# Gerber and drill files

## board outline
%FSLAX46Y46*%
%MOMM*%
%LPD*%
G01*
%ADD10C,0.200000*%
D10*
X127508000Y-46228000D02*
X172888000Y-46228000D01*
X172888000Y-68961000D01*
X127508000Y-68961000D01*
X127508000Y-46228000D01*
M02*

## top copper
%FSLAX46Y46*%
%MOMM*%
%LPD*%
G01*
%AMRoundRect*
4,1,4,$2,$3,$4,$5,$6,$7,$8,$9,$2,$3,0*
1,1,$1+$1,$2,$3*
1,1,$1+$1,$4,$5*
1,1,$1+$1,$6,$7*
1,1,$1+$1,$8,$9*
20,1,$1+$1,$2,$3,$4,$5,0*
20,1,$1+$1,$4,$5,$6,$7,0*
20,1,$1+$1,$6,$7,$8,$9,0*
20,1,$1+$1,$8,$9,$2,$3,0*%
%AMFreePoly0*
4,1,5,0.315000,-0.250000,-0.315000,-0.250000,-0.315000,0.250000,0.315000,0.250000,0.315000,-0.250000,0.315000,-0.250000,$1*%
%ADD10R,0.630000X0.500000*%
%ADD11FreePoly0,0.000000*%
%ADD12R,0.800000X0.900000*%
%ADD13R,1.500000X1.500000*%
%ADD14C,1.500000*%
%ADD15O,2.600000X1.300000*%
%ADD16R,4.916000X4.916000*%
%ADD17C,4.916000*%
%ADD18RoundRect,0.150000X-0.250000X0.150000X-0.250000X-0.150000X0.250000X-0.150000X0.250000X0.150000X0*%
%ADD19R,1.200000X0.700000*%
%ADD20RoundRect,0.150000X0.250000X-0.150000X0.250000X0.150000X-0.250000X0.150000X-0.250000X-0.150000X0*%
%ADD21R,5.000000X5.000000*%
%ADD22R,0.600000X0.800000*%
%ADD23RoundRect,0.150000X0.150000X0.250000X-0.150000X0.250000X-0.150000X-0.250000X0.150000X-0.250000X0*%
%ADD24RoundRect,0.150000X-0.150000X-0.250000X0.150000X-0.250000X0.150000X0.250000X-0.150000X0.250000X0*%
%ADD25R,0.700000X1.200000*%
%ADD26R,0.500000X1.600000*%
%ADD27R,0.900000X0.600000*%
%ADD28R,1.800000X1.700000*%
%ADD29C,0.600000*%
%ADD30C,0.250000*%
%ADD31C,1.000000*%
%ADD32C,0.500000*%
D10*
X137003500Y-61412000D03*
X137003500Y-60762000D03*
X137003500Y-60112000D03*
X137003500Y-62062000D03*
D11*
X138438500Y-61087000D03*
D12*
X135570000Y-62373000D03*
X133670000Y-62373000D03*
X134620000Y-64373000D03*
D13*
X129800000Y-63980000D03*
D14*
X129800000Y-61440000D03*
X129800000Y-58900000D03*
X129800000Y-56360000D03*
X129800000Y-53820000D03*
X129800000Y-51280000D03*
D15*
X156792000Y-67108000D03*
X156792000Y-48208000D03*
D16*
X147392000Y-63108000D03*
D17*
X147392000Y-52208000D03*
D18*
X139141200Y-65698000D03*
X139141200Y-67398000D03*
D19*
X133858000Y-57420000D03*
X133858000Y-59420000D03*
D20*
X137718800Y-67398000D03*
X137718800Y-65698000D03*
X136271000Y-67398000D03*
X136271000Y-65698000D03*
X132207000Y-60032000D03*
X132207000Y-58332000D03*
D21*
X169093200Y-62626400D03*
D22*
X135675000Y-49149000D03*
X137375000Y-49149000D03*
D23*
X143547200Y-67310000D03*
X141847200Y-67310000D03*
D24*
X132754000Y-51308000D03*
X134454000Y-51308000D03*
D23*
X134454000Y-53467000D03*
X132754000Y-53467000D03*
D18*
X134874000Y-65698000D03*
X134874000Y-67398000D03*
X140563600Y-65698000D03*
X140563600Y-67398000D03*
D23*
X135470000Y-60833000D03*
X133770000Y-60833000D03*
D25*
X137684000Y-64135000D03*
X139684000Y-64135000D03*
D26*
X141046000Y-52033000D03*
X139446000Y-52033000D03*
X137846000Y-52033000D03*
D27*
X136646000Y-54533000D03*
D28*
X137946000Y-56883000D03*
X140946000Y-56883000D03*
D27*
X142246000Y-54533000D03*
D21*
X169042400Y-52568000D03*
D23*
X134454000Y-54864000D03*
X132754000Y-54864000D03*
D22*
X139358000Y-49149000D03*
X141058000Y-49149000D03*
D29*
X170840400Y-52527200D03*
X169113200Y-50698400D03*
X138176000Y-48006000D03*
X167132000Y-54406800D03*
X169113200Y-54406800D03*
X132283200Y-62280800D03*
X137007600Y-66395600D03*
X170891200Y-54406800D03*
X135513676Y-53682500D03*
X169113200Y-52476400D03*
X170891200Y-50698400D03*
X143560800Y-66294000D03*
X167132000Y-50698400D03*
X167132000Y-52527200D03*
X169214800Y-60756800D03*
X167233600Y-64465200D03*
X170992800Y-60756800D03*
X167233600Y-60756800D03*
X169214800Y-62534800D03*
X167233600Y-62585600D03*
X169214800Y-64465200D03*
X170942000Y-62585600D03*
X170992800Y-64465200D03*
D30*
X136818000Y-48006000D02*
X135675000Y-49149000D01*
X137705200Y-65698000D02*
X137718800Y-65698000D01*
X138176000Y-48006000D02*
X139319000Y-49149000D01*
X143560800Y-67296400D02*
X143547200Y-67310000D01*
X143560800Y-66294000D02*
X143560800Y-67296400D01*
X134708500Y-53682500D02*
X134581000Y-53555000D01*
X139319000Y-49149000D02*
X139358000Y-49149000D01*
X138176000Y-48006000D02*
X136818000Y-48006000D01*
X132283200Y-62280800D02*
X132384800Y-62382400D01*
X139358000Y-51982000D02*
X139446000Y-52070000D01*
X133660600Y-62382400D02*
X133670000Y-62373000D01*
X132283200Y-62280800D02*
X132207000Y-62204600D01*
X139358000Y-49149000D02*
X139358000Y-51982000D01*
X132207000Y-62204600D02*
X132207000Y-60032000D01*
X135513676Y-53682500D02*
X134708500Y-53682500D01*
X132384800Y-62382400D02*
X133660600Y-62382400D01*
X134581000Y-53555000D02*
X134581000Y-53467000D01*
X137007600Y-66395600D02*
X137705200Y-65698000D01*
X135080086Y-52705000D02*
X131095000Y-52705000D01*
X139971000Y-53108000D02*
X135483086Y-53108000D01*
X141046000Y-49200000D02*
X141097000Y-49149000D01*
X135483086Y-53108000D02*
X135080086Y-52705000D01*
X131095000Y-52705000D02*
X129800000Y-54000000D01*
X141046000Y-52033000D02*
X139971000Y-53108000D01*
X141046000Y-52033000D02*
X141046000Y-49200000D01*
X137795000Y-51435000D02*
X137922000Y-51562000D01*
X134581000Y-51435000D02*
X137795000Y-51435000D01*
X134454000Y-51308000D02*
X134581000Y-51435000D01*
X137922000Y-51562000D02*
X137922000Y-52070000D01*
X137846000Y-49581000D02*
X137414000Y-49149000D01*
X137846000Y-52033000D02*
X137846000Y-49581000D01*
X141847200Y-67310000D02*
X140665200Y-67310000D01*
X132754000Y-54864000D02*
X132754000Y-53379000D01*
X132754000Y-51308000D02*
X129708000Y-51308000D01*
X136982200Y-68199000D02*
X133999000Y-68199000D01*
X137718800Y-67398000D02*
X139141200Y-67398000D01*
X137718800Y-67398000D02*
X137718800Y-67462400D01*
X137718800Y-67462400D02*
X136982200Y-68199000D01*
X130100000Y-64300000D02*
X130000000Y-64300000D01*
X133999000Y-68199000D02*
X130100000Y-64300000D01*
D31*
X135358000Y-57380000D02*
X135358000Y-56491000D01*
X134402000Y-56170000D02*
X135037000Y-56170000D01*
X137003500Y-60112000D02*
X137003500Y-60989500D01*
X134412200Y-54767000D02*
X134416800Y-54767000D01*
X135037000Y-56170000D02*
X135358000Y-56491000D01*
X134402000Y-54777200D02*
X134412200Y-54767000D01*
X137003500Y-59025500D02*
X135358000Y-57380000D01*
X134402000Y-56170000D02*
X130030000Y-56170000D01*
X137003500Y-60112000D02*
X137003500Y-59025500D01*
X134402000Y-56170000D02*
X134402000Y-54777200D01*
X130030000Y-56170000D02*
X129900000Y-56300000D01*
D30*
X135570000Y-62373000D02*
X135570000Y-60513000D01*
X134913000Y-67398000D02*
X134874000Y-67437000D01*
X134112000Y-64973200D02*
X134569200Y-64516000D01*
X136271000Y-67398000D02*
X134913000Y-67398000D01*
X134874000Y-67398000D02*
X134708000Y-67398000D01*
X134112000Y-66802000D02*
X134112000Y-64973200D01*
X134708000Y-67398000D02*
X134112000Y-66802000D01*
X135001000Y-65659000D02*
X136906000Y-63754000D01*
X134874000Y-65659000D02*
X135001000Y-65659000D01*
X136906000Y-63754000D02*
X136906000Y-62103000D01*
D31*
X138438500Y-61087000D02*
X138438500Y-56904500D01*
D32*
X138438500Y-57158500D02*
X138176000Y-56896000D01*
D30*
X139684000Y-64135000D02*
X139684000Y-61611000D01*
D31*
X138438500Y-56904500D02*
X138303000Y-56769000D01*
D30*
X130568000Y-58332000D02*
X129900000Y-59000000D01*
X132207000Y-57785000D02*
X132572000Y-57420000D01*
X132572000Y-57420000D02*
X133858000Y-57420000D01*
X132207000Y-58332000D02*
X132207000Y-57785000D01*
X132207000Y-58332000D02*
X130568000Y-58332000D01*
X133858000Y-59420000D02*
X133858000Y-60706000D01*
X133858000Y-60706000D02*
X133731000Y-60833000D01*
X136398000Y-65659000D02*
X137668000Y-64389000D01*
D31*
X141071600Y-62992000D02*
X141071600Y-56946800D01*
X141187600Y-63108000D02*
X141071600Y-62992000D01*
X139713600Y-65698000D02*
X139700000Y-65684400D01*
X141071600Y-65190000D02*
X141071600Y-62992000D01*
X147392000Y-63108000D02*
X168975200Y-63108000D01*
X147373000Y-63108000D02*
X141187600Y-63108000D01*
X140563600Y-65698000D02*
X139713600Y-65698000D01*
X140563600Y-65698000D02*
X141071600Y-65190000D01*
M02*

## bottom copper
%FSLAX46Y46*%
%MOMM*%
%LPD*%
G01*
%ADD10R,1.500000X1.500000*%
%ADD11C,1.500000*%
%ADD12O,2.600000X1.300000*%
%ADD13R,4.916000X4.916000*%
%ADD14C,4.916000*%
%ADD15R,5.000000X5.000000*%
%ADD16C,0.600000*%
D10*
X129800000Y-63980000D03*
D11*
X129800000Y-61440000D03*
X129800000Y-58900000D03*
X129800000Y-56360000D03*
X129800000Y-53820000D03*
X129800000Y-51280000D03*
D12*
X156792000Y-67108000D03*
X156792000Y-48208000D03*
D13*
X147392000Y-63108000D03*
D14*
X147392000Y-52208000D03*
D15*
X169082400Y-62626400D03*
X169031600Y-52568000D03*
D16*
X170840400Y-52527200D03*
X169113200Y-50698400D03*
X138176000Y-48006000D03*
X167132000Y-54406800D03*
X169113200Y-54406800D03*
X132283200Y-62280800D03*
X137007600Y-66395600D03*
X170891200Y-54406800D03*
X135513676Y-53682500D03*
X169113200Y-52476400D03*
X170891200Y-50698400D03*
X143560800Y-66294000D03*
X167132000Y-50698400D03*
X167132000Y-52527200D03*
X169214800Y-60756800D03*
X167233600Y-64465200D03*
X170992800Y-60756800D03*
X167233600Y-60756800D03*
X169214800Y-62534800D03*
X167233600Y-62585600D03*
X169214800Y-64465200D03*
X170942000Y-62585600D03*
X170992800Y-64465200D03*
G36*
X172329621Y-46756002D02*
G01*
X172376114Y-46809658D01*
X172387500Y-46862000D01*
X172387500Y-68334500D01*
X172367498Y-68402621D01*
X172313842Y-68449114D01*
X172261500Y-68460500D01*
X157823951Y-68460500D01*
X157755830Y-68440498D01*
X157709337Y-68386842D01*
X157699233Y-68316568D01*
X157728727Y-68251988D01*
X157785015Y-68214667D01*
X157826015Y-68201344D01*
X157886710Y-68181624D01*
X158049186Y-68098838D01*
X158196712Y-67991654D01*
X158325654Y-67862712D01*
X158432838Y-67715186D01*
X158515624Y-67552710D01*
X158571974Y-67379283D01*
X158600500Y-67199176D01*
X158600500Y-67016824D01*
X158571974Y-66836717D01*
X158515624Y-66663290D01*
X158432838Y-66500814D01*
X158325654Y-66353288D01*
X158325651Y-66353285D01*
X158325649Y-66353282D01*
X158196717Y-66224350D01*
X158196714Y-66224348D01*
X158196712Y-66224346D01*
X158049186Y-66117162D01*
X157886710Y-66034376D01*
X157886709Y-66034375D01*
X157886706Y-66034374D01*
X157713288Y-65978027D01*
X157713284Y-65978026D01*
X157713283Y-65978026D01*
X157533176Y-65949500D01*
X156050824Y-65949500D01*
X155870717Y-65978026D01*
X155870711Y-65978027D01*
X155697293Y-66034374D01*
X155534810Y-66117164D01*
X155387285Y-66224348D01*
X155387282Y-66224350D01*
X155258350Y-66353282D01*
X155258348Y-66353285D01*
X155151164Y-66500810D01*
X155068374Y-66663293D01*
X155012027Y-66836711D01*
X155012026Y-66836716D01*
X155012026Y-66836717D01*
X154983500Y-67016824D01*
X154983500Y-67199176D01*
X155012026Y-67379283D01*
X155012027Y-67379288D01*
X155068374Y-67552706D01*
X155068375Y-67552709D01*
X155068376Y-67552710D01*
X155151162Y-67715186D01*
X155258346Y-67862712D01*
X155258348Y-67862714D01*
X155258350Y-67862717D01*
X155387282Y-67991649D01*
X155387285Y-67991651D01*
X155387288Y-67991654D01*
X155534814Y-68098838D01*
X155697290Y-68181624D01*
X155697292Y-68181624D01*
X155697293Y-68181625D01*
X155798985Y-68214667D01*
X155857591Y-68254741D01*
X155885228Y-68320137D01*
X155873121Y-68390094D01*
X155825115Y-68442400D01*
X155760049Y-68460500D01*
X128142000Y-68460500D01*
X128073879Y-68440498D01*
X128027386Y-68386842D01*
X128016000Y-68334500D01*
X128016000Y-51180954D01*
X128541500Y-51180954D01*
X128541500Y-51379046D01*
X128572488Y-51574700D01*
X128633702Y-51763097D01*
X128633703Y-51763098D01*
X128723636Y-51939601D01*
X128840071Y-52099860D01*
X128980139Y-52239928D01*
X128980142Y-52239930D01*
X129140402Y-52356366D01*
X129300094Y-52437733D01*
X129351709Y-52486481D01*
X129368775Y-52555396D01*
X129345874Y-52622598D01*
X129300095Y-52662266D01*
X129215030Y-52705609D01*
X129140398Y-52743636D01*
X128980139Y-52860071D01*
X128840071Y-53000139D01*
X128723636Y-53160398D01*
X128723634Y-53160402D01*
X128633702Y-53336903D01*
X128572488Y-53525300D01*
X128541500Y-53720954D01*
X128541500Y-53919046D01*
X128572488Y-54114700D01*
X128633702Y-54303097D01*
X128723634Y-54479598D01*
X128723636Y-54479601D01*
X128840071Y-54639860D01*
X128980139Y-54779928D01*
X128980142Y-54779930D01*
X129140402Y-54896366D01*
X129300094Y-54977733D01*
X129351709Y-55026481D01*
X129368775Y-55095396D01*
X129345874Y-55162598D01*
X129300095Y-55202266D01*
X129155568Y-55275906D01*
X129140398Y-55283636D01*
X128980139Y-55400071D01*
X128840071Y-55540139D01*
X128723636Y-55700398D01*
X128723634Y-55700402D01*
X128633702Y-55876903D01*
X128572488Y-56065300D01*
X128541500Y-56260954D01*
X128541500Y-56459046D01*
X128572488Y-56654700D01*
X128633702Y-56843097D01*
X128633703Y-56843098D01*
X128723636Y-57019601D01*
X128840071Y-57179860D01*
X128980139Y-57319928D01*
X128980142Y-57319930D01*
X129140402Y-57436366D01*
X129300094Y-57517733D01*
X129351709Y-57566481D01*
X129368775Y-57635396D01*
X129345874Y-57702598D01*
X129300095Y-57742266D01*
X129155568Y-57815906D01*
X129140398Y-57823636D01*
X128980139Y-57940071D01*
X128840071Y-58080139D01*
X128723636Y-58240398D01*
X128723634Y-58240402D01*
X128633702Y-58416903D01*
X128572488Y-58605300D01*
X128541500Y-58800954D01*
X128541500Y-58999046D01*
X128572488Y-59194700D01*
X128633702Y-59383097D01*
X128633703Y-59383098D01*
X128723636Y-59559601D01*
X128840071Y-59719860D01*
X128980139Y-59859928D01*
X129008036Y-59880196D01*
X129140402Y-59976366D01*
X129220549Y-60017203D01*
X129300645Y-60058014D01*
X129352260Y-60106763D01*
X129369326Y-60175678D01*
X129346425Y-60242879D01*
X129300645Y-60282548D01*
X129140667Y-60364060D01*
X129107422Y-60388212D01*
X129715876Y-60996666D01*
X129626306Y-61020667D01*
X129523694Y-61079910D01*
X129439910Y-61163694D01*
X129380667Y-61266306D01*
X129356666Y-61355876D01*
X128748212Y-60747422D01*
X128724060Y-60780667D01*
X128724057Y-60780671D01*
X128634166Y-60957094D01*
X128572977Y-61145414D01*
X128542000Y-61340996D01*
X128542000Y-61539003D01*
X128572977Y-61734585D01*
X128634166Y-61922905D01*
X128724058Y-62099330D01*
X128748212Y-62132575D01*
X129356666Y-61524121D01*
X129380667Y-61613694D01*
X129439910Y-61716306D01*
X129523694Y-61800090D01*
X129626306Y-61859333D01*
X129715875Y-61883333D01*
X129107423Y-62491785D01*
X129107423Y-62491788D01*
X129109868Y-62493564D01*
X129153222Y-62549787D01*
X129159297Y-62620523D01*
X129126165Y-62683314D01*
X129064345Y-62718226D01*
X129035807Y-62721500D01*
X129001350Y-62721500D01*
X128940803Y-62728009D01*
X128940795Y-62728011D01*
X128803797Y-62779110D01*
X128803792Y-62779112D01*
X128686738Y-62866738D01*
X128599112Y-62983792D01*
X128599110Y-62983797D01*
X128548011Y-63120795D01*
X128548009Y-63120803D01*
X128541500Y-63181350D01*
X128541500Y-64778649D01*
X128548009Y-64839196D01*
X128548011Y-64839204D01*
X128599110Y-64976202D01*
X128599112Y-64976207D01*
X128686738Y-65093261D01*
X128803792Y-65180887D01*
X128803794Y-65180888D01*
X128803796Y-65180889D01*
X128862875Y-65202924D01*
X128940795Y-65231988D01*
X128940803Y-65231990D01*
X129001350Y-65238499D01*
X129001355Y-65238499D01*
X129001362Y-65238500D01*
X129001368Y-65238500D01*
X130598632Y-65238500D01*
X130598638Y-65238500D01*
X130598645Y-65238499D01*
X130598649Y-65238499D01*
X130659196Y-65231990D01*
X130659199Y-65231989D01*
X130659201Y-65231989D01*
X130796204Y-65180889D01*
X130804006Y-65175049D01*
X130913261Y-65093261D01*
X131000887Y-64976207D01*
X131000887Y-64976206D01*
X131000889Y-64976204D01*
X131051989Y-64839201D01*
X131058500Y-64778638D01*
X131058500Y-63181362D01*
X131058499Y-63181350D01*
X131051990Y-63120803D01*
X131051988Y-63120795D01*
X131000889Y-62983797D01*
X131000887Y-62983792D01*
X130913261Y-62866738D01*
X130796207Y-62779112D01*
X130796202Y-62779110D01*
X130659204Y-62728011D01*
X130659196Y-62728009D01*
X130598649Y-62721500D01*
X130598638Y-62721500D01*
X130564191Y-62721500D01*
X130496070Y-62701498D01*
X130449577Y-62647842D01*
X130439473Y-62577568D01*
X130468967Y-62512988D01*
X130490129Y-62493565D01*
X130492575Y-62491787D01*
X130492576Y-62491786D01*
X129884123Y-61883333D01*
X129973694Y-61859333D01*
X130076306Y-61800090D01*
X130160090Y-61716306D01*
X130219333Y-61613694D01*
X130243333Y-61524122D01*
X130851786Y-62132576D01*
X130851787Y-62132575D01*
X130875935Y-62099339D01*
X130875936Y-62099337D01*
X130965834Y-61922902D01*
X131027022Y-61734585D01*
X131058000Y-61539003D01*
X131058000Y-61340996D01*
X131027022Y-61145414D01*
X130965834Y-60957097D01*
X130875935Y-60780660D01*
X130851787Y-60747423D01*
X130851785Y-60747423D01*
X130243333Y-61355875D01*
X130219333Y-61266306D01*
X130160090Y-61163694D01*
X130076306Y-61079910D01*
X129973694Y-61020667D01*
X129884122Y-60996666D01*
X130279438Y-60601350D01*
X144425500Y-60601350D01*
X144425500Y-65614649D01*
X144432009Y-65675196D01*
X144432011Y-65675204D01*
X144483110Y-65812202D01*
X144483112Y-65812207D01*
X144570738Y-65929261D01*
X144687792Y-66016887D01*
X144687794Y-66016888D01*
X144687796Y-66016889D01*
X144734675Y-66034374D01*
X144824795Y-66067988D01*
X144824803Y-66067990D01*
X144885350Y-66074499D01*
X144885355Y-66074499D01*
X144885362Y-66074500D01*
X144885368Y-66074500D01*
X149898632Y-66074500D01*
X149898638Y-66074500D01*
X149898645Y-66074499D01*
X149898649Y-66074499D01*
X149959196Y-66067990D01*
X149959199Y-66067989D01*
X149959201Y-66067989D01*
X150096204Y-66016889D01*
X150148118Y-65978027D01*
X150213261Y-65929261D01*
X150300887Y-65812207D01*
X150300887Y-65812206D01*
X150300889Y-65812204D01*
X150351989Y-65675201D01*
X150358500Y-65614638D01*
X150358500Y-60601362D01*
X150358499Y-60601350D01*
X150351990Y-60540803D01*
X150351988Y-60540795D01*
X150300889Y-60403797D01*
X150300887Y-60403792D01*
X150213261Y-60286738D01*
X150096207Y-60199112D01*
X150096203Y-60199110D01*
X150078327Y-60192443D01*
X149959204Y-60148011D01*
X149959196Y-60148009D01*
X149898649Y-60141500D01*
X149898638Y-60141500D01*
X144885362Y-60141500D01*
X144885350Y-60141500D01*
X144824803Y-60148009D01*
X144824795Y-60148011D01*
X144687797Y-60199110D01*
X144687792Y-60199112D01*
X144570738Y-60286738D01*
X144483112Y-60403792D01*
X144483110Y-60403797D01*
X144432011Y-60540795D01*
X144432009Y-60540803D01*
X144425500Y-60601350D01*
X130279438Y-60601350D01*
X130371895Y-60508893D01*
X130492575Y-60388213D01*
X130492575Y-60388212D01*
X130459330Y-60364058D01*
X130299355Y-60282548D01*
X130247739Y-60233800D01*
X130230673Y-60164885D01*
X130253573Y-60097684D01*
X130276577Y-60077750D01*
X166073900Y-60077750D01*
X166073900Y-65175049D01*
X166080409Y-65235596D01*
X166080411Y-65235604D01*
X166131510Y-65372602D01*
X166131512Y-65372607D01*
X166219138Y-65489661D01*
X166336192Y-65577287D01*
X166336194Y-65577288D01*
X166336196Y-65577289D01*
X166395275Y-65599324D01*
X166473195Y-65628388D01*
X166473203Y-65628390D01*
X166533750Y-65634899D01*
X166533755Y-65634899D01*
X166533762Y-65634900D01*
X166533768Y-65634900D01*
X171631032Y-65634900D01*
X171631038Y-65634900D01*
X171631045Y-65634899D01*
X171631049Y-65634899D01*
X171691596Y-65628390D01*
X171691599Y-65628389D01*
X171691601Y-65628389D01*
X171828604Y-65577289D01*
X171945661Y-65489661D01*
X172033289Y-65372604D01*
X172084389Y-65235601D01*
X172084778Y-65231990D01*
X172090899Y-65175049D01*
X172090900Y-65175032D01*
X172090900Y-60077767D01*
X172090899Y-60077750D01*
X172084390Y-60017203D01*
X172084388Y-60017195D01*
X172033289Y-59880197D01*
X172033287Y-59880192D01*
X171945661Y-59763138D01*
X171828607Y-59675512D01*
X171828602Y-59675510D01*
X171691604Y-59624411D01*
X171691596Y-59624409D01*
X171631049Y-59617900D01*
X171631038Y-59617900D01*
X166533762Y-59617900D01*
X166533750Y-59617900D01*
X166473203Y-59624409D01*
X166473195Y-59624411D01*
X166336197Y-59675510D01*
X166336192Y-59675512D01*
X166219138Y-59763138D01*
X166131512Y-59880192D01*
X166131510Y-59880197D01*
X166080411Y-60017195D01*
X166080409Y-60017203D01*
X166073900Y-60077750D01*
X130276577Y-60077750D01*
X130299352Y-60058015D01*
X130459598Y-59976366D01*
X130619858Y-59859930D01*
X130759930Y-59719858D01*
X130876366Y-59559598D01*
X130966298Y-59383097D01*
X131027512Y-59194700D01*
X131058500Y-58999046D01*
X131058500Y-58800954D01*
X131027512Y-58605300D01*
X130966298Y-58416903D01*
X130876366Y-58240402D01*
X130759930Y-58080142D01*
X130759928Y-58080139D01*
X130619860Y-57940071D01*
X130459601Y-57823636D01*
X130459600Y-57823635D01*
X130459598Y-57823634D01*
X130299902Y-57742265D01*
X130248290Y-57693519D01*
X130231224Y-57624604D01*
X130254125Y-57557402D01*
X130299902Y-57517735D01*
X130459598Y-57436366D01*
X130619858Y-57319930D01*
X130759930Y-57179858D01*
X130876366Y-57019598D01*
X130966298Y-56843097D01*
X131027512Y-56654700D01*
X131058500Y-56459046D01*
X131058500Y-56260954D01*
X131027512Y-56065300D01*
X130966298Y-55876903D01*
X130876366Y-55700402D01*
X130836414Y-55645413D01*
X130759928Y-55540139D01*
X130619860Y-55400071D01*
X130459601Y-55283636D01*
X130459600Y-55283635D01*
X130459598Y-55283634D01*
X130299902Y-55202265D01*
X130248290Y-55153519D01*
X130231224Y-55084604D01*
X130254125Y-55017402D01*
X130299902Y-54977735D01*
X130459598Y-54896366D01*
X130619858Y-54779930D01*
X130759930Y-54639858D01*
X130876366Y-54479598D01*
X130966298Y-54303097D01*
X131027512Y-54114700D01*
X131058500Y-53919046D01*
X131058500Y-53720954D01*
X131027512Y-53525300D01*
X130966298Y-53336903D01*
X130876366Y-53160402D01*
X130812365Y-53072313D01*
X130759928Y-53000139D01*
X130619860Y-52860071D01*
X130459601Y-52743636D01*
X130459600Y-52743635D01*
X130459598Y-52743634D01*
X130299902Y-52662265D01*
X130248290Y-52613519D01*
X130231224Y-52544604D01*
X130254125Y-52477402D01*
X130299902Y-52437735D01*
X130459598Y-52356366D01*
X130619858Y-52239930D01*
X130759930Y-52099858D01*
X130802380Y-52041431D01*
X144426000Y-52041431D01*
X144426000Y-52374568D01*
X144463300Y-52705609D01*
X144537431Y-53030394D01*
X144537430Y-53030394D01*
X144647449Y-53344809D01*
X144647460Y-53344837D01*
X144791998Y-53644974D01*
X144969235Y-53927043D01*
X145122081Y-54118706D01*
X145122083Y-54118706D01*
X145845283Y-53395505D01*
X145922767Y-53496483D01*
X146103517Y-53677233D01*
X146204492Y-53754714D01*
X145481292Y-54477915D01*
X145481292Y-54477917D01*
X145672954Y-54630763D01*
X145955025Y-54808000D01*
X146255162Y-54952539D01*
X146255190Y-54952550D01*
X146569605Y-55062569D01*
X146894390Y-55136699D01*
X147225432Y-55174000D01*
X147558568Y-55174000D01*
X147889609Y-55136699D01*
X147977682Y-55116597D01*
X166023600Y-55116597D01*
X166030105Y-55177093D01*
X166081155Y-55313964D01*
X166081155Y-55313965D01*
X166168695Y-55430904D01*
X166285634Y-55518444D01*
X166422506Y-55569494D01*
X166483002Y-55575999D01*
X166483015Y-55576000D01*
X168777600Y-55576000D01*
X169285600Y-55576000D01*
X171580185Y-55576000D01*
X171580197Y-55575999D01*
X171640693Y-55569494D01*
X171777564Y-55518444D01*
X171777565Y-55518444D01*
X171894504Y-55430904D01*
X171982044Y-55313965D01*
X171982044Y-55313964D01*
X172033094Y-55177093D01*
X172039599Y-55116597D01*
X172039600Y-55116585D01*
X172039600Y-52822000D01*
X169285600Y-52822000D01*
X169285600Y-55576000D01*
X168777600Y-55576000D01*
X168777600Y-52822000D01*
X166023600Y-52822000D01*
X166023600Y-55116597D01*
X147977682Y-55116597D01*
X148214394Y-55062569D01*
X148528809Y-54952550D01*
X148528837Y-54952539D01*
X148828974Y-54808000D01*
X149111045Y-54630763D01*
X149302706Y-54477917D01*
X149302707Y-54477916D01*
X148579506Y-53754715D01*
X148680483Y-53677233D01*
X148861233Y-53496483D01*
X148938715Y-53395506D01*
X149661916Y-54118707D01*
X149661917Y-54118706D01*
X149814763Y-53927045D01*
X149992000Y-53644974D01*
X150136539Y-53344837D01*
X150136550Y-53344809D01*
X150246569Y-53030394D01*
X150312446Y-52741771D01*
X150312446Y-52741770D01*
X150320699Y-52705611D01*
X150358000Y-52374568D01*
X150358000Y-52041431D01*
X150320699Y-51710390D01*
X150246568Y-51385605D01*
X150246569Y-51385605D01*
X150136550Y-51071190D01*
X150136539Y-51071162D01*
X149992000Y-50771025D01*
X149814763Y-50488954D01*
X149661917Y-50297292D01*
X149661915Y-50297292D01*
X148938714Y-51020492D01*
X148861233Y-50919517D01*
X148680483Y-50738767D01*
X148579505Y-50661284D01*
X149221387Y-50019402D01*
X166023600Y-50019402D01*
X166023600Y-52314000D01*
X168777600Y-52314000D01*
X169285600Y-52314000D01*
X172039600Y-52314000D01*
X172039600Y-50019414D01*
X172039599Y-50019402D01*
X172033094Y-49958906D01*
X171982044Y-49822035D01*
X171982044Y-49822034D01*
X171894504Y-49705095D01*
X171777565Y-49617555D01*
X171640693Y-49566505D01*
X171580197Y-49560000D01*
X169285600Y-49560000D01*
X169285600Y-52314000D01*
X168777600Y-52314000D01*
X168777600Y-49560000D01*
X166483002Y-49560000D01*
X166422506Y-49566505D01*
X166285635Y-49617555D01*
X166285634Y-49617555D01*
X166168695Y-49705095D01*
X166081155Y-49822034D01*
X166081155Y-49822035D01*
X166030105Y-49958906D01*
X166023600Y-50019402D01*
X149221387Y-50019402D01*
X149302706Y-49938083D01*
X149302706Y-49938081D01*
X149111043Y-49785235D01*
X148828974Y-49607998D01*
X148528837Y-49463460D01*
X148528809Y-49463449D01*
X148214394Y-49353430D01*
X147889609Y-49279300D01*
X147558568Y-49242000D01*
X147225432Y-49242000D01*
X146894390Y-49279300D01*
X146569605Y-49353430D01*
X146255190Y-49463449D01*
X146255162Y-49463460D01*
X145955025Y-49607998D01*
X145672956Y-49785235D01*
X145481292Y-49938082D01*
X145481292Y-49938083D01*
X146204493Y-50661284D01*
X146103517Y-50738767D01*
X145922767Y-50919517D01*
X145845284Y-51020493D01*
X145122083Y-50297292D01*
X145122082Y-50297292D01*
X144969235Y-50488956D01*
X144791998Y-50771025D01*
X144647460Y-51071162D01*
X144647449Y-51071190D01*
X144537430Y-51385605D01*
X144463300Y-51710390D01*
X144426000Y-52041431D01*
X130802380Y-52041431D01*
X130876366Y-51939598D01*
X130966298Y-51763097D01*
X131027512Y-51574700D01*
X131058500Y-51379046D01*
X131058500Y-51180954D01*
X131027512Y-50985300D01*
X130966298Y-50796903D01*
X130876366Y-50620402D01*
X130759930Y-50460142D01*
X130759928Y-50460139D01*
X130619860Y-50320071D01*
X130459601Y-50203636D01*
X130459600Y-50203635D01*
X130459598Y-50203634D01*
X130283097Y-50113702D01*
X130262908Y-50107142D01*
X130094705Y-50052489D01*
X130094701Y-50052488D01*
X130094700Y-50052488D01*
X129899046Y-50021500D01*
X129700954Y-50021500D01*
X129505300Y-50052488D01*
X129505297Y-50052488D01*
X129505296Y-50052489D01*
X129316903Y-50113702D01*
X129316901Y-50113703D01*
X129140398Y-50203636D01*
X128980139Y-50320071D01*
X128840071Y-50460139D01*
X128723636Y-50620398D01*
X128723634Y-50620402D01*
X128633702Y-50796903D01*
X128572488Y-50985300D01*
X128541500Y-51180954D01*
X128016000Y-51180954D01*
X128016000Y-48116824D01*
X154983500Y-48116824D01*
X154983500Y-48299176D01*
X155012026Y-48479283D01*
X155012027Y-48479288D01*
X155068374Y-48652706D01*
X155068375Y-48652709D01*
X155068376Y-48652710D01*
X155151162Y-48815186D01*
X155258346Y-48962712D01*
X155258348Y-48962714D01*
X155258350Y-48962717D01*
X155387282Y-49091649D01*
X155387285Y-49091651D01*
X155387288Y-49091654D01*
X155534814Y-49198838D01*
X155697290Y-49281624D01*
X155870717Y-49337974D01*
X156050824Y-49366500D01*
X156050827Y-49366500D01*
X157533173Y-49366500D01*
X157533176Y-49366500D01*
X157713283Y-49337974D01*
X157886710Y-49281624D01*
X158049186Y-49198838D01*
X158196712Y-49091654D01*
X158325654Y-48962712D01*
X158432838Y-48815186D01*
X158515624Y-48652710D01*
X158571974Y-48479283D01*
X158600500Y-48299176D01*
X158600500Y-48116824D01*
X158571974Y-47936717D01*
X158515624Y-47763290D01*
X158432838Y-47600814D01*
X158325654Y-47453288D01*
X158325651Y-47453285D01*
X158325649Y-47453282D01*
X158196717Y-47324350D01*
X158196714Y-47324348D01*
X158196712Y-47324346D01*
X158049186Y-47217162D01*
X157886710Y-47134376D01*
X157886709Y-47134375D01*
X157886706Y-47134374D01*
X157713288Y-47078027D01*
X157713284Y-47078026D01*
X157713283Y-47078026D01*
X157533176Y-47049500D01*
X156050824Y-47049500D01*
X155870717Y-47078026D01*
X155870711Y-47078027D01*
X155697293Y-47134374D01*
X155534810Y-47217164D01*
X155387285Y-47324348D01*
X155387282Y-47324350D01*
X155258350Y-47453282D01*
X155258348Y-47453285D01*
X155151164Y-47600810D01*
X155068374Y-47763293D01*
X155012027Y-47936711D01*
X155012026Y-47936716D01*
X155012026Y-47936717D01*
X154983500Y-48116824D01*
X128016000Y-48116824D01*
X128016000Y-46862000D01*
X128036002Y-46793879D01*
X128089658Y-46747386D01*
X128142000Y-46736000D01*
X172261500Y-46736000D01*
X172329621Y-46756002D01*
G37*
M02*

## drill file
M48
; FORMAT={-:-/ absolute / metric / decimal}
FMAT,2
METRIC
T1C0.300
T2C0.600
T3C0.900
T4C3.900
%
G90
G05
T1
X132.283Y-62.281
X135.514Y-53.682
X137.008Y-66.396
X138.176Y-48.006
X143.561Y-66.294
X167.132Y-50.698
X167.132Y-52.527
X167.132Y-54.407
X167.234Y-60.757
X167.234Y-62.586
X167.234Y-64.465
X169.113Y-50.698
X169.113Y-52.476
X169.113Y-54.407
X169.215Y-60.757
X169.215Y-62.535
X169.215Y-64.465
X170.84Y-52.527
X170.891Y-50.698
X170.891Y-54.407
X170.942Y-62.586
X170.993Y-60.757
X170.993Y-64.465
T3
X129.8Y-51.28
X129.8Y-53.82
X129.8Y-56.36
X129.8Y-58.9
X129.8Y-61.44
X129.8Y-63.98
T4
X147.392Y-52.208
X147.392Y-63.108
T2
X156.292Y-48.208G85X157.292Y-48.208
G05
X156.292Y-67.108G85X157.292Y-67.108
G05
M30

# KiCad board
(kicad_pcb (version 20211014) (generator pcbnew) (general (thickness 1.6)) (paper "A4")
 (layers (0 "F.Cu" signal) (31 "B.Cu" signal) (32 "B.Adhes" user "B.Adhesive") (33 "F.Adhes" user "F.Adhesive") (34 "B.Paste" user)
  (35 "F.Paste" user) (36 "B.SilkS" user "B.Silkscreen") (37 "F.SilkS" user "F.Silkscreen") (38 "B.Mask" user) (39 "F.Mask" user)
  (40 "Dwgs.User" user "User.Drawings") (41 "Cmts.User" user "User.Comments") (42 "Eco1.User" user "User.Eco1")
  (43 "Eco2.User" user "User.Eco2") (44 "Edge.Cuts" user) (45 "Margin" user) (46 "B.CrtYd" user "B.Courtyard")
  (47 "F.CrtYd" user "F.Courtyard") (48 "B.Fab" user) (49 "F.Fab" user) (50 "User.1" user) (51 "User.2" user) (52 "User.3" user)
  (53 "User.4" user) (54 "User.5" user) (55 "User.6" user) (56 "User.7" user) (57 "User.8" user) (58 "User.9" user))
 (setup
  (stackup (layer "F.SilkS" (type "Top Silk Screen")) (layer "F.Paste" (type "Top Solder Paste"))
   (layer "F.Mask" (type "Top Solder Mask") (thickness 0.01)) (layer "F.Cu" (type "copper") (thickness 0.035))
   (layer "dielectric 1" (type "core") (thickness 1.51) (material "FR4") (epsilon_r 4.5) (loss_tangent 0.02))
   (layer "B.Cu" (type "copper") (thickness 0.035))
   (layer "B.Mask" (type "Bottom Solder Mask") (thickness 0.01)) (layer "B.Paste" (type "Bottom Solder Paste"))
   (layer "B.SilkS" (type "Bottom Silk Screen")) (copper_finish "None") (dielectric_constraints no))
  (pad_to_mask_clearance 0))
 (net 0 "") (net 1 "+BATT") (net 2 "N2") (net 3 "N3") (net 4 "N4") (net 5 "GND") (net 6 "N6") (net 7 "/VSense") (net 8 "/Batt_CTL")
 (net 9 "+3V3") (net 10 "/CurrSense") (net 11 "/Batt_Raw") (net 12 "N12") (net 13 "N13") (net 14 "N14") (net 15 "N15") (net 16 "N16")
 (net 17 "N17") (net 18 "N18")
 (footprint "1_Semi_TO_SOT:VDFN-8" (layer "F.Cu") (at 138.4385 61.087) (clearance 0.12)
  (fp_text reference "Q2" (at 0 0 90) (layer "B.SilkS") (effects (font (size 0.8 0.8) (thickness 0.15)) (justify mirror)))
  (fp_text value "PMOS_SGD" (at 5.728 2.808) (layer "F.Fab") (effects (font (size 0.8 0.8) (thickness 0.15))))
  (pad "1" smd rect (at -1.435 0.325) (size 0.63 0.5) (layers "F.Cu" "F.Mask") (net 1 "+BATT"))
  (pad "1" smd rect (at -1.435 -0.325) (size 0.63 0.5) (layers "F.Cu" "F.Mask") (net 1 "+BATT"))
  (pad "1" smd rect (at -1.435 -0.975) (size 0.63 0.5) (layers "F.Cu" "F.Mask") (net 1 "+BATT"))
  (pad "2" smd rect (at -1.435 0.975) (size 0.63 0.5) (layers "F.Cu" "F.Mask") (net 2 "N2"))
  (pad "3" smd custom (at 0 0) (size 0.63 0.5) (layers "F.Cu") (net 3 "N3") (zone_connect 0) (options (clearance outline) (anchor rect))
   (primitives)))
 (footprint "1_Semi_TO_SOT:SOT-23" (layer "F.Cu") (at 134.62 63.373 -90)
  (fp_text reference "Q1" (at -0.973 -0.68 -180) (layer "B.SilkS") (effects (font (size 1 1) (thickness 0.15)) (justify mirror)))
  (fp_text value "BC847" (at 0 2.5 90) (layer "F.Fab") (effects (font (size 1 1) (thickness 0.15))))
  (pad "1" smd rect locked (at -1 -0.95 270) (size 0.9 0.8) (layers "F.Cu" "F.Paste" "F.Mask") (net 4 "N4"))
  (pad "2" smd rect locked (at -1 0.95 270) (size 0.9 0.8) (layers "F.Cu" "F.Paste" "F.Mask") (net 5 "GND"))
  (pad "3" smd rect locked (at 1 0 270) (size 0.9 0.8) (layers "F.Cu" "F.Paste" "F.Mask") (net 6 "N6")))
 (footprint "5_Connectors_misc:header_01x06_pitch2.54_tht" (layer "F.Cu") (at 129.8 63.98 90)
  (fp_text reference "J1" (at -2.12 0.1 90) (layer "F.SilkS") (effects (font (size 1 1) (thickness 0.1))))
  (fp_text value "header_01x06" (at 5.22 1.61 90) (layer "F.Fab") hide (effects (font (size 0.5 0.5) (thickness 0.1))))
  (pad "1" thru_hole rect locked (at 0 0 90) (size 1.5 1.5) (drill 0.9) (layers *.Cu *.Mask) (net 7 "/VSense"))
  (pad "2" thru_hole circle locked (at 2.54 0 90) (size 1.5 1.5) (drill 0.9) (layers *.Cu *.Mask) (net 5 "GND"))
  (pad "3" thru_hole circle locked (at 5.08 0 90) (size 1.5 1.5) (drill 0.9) (layers *.Cu *.Mask) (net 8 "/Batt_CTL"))
  (pad "4" thru_hole circle locked (at 7.62 0 90) (size 1.5 1.5) (drill 0.9) (layers *.Cu *.Mask) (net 1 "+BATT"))
  (pad "5" thru_hole circle locked (at 10.16 0 90) (size 1.5 1.5) (drill 0.9) (layers *.Cu *.Mask) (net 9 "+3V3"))
  (pad "6" thru_hole circle locked (at 12.7 0 90) (size 1.5 1.5) (drill 0.9) (layers *.Cu *.Mask) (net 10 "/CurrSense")))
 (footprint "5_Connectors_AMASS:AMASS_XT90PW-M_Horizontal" (layer "F.Cu") (at 156.792 57.658 90)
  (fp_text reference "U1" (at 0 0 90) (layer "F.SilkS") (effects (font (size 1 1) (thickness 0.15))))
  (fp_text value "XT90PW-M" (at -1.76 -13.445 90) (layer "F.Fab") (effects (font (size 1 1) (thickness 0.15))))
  (pad "" thru_hole oval (at -9.45 0 90) (size 1.3 2.6) (drill oval 0.6 1.6) (layers *.Cu *.Mask))
  (pad "" thru_hole oval (at 9.45 0 90) (size 1.3 2.6) (drill oval 0.6 1.6) (layers *.Cu *.Mask))
  (pad "1" thru_hole rect (at -5.45 -9.4 90) (size 4.916 4.916) (drill 3.9) (layers *.Cu *.Mask) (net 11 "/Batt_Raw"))
  (pad "2" thru_hole circle (at 5.45 -9.4 90) (size 4.916 4.916) (drill 3.9) (layers *.Cu *.Mask) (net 5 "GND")))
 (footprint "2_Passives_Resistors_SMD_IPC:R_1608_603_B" (layer "F.Cu") (at 139.1412 66.548 -90)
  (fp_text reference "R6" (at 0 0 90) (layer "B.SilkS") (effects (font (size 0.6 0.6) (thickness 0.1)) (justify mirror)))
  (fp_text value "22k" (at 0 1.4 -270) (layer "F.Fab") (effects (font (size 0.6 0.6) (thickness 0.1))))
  (pad "1" smd roundrect (at -0.85 0 270) (size 0.6 0.8) (layers "F.Cu" "F.Paste" "F.Mask") (roundrect_rratio 0.25) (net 11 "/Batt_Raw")
   (thermal_width 0.15) (thermal_gap 0.15))
  (pad "2" smd roundrect (at 0.85 0 270) (size 0.6 0.8) (layers "F.Cu" "F.Paste" "F.Mask") (roundrect_rratio 0.25) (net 7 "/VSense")
   (thermal_width 0.15) (thermal_gap 0.15)))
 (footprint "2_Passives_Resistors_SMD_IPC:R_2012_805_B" (layer "F.Cu") (at 133.858 58.42 -90)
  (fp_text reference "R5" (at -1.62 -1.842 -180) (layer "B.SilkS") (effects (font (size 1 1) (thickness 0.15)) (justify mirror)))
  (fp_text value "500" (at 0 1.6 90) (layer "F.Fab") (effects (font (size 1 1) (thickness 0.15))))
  (pad "1" smd rect locked (at -1 0 270) (size 0.7 1.2) (layers "F.Cu" "F.Paste" "F.Mask") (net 8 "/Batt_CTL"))
  (pad "2" smd rect locked (at 1 0 270) (size 0.7 1.2) (layers "F.Cu" "F.Paste" "F.Mask") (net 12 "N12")))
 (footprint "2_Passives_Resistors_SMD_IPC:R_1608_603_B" (layer "F.Cu") (at 137.7188 66.548 90)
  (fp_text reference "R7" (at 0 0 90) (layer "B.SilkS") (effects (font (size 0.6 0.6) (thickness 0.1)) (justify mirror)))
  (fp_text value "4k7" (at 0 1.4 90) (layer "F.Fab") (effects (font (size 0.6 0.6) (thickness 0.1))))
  (pad "1" smd roundrect (at -0.85 0 90) (size 0.6 0.8) (layers "F.Cu" "F.Paste" "F.Mask") (roundrect_rratio 0.25) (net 7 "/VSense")
   (thermal_width 0.15) (thermal_gap 0.15))
  (pad "2" smd roundrect (at 0.85 0 90) (size 0.6 0.8) (layers "F.Cu" "F.Paste" "F.Mask") (roundrect_rratio 0.25) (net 5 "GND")
   (thermal_width 0.15) (thermal_gap 0.15)))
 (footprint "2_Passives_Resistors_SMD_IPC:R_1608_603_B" (layer "F.Cu") (at 136.271 66.548 90)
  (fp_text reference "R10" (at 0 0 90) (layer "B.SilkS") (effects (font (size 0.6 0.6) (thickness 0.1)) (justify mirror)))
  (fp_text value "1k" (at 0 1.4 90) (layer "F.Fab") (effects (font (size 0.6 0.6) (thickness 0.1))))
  (pad "1" smd roundrect (at -0.85 0 90) (size 0.6 0.8) (layers "F.Cu" "F.Paste" "F.Mask") (roundrect_rratio 0.25) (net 6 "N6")
   (thermal_width 0.15) (thermal_gap 0.15))
  (pad "2" smd roundrect (at 0.85 0 90) (size 0.6 0.8) (layers "F.Cu" "F.Paste" "F.Mask") (roundrect_rratio 0.25) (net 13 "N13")
   (thermal_width 0.15) (thermal_gap 0.15)))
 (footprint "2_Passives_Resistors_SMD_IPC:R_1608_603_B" (layer "F.Cu") (at 132.207 59.182 90)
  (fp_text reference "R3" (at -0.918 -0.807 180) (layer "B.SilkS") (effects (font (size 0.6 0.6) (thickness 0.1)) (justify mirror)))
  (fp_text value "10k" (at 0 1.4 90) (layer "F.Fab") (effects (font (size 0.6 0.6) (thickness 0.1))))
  (pad "1" smd roundrect (at -0.85 0 90) (size 0.6 0.8) (layers "F.Cu" "F.Paste" "F.Mask") (roundrect_rratio 0.25) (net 5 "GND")
   (thermal_width 0.15) (thermal_gap 0.15))
  (pad "2" smd roundrect (at 0.85 0 90) (size 0.6 0.8) (layers "F.Cu" "F.Paste" "F.Mask") (roundrect_rratio 0.25) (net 8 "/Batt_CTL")
   (thermal_width 0.15) (thermal_gap 0.15)))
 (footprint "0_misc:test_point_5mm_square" (layer "F.Cu") (at 169.1132 62.6364)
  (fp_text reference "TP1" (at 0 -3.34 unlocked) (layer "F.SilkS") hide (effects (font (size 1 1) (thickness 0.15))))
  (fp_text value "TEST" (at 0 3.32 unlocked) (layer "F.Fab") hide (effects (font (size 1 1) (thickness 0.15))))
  (pad "1" smd rect (at -0.02 -0.01) (size 5 5) (layers "F.Cu" "F.Paste" "F.Mask") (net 11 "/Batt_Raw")))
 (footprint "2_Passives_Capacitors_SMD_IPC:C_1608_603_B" (layer "F.Cu") (at 136.525 49.149)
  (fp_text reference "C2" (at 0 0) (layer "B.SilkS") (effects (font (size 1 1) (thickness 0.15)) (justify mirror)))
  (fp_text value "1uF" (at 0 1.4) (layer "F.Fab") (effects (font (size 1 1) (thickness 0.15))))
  (pad "1" smd rect (at -0.85 0) (size 0.6 0.8) (layers "F.Cu" "F.Paste" "F.Mask") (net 5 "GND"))
  (pad "2" smd rect (at 0.85 0) (size 0.6 0.8) (layers "F.Cu" "F.Paste" "F.Mask") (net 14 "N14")))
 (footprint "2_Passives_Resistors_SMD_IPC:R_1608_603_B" (layer "F.Cu") (at 142.6972 67.31 180)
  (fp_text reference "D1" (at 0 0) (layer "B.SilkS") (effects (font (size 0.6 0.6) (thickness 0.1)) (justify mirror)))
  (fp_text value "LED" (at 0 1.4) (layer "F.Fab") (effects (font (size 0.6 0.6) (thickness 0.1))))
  (pad "1" smd roundrect (at -0.85 0 180) (size 0.6 0.8) (layers "F.Cu" "F.Paste" "F.Mask") (roundrect_rratio 0.25) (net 5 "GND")
   (thermal_width 0.15) (thermal_gap 0.15))
  (pad "2" smd roundrect (at 0.85 0 180) (size 0.6 0.8) (layers "F.Cu" "F.Paste" "F.Mask") (roundrect_rratio 0.25) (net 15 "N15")
   (thermal_width 0.15) (thermal_gap 0.15)))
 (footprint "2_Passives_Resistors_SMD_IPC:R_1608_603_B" (layer "F.Cu") (at 133.604 51.308)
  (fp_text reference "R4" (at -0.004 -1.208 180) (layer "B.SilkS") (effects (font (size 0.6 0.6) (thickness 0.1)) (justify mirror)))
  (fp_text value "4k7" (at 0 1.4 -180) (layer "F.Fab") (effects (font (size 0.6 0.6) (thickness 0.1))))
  (pad "1" smd roundrect (at -0.85 0) (size 0.6 0.8) (layers "F.Cu" "F.Paste" "F.Mask") (roundrect_rratio 0.25) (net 10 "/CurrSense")
   (thermal_width 0.15) (thermal_gap 0.15))
  (pad "2" smd roundrect (at 0.85 0) (size 0.6 0.8) (layers "F.Cu" "F.Paste" "F.Mask") (roundrect_rratio 0.25) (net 14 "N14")
   (thermal_width 0.15) (thermal_gap 0.15)))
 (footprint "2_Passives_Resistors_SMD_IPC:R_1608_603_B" (layer "F.Cu") (at 133.604 53.467 180)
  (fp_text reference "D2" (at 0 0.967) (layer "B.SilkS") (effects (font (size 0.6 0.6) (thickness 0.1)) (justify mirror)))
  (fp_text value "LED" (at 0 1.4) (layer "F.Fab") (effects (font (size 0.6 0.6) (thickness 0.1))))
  (pad "1" smd roundrect (at -0.85 0 180) (size 0.6 0.8) (layers "F.Cu" "F.Paste" "F.Mask") (roundrect_rratio 0.25) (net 5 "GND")
   (thermal_width 0.15) (thermal_gap 0.15))
  (pad "2" smd roundrect (at 0.85 0 180) (size 0.6 0.8) (layers "F.Cu" "F.Paste" "F.Mask") (roundrect_rratio 0.25) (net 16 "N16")
   (thermal_width 0.15) (thermal_gap 0.15)))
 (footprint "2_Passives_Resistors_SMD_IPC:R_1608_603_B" (layer "F.Cu") (at 134.874 66.548 -90)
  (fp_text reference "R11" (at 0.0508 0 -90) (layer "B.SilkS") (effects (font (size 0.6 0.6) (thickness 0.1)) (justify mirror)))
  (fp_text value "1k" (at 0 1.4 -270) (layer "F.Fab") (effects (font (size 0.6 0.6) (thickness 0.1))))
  (pad "1" smd roundrect (at -0.85 0 270) (size 0.6 0.8) (layers "F.Cu" "F.Paste" "F.Mask") (roundrect_rratio 0.25) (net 2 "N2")
   (thermal_width 0.15) (thermal_gap 0.15))
  (pad "2" smd roundrect (at 0.85 0 270) (size 0.6 0.8) (layers "F.Cu" "F.Paste" "F.Mask") (roundrect_rratio 0.25) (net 6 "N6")
   (thermal_width 0.15) (thermal_gap 0.15)))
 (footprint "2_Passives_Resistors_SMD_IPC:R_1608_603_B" (layer "F.Cu") (at 140.5636 66.548 -90)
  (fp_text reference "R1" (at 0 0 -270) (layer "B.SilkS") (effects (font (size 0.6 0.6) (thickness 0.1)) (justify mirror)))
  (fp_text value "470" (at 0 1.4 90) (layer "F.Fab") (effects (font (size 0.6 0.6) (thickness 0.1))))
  (pad "1" smd roundrect (at -0.85 0 270) (size 0.6 0.8) (layers "F.Cu" "F.Paste" "F.Mask") (roundrect_rratio 0.25) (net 11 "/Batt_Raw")
   (thermal_width 0.15) (thermal_gap 0.15))
  (pad "2" smd roundrect (at 0.85 0 270) (size 0.6 0.8) (layers "F.Cu" "F.Paste" "F.Mask") (roundrect_rratio 0.25) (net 15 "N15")
   (thermal_width 0.15) (thermal_gap 0.15)))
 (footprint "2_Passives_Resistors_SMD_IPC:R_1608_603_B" (layer "F.Cu") (at 134.62 60.833 180)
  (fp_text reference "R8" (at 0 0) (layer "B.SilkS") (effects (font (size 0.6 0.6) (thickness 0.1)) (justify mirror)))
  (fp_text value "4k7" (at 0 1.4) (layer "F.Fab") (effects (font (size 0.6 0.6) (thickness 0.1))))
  (pad "1" smd roundrect (at -0.85 0 180) (size 0.6 0.8) (layers "F.Cu" "F.Paste" "F.Mask") (roundrect_rratio 0.25) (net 4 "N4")
   (thermal_width 0.15) (thermal_gap 0.15))
  (pad "2" smd roundrect (at 0.85 0 180) (size 0.6 0.8) (layers "F.Cu" "F.Paste" "F.Mask") (roundrect_rratio 0.25) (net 12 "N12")
   (thermal_width 0.15) (thermal_gap 0.15)))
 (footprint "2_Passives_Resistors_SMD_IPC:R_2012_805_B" (layer "F.Cu") (at 138.684 64.135)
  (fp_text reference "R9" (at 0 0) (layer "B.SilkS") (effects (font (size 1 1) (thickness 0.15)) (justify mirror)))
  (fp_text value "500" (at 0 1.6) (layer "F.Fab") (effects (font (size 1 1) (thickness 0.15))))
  (pad "1" smd rect locked (at -1 0) (size 0.7 1.2) (layers "F.Cu" "F.Paste" "F.Mask") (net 13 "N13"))
  (pad "2" smd rect locked (at 1 0) (size 0.7 1.2) (layers "F.Cu" "F.Paste" "F.Mask") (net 3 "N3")))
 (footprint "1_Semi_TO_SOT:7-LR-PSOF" (layer "F.Cu") (at 139.446 54.483 180) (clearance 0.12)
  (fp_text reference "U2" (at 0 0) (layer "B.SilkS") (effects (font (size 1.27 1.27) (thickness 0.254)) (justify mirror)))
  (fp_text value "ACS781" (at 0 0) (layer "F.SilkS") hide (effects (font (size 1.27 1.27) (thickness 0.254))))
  (pad "1" smd rect (at -1.6 2.45 180) (size 0.5 1.6) (layers "F.Cu" "F.Paste" "F.Mask") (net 9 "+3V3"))
  (pad "2" smd rect (at 0 2.45 180) (size 0.5 1.6) (layers "F.Cu" "F.Paste" "F.Mask") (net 5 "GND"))
  (pad "3" smd rect (at 1.6 2.45 180) (size 0.5 1.6) (layers "F.Cu" "F.Paste" "F.Mask") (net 14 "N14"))
  (pad "4" smd rect (at 2.8 -0.05 270) (size 0.6 0.9) (layers "F.Cu" "F.Paste" "F.Mask") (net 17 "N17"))
  (pad "5" smd rect (at 1.5 -2.4 270) (size 1.7 1.8) (layers "F.Cu" "F.Paste" "F.Mask") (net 3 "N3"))
  (pad "6" smd rect (at -1.5 -2.4 270) (size 1.7 1.8) (layers "F.Cu" "F.Paste" "F.Mask") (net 11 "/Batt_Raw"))
  (pad "7" smd rect (at -2.8 -0.05 270) (size 0.6 0.9) (layers "F.Cu" "F.Paste" "F.Mask") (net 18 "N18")))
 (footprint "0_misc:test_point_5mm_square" (layer "F.Cu") (at 169.0624 52.578)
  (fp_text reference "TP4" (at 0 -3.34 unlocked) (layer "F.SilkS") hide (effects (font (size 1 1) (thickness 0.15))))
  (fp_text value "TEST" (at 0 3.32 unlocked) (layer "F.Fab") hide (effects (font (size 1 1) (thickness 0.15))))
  (pad "1" smd rect (at -0.02 -0.01) (size 5 5) (layers "F.Cu" "F.Paste" "F.Mask") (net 5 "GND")))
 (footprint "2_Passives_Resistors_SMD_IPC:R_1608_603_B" (layer "F.Cu") (at 133.604 54.864 180)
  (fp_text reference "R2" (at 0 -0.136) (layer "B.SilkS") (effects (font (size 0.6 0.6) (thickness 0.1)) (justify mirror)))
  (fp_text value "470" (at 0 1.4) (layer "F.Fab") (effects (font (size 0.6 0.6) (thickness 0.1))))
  (pad "1" smd roundrect (at -0.85 0 180) (size 0.6 0.8) (layers "F.Cu" "F.Paste" "F.Mask") (roundrect_rratio 0.25) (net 1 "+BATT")
   (thermal_width 0.15) (thermal_gap 0.15))
  (pad "2" smd roundrect (at 0.85 0 180) (size 0.6 0.8) (layers "F.Cu" "F.Paste" "F.Mask") (roundrect_rratio 0.25) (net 16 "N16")
   (thermal_width 0.15) (thermal_gap 0.15)))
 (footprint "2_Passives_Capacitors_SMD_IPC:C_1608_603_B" (layer "F.Cu") (at 140.208 49.149)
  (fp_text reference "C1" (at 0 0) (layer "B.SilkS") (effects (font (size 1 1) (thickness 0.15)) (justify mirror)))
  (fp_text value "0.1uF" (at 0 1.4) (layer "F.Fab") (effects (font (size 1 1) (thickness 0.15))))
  (pad "1" smd rect (at -0.85 0) (size 0.6 0.8) (layers "F.Cu" "F.Paste" "F.Mask") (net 5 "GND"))
  (pad "2" smd rect (at 0.85 0) (size 0.6 0.8) (layers "F.Cu" "F.Paste" "F.Mask") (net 9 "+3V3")))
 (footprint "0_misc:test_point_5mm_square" (layer "B.Cu") (at 169.0624 62.6364 180)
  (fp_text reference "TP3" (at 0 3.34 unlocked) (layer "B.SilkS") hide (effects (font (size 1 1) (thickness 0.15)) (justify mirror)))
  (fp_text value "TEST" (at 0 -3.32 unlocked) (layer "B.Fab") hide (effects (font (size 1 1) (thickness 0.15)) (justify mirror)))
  (pad "1" smd rect (at -0.02 0.01 180) (size 5 5) (layers "B.Cu" "B.Paste" "B.Mask") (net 11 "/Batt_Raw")))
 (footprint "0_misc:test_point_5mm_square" (layer "B.Cu") (at 169.0116 52.578 180)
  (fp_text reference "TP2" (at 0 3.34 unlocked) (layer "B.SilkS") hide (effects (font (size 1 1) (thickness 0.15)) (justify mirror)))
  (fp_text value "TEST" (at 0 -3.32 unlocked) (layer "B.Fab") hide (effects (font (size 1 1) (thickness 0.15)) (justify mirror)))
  (pad "1" smd rect (at -0.02 0.01 180) (size 5 5) (layers "B.Cu" "B.Paste" "B.Mask") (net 5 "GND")))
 (gr_rect (start 127.508 46.228) (end 172.888 68.961) (layer "Edge.Cuts") (width 0.2) (fill none))
 (segment (start 136.818 48.006) (end 135.675 49.149) (width 0.25) (layer "F.Cu") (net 5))
 (segment (start 137.7052 65.698) (end 137.7188 65.698) (width 0.25) (layer "F.Cu") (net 5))
 (segment (start 138.176 48.006) (end 139.319 49.149) (width 0.25) (layer "F.Cu") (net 5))
 (segment (start 143.5608 67.2964) (end 143.5472 67.31) (width 0.25) (layer "F.Cu") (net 5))
 (segment (start 143.5608 66.294) (end 143.5608 67.2964) (width 0.25) (layer "F.Cu") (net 5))
 (segment (start 134.7085 53.6825) (end 134.581 53.555) (width 0.25) (layer "F.Cu") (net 5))
 (segment (start 139.319 49.149) (end 139.358 49.149) (width 0.25) (layer "F.Cu") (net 5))
 (segment (start 138.176 48.006) (end 136.818 48.006) (width 0.25) (layer "F.Cu") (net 5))
 (segment (start 132.2832 62.2808) (end 132.3848 62.3824) (width 0.25) (layer "F.Cu") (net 5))
 (segment (start 139.358 51.982) (end 139.446 52.07) (width 0.25) (layer "F.Cu") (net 5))
 (segment (start 133.6606 62.3824) (end 133.67 62.373) (width 0.25) (layer "F.Cu") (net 5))
 (segment (start 132.2832 62.2808) (end 132.207 62.2046) (width 0.25) (layer "F.Cu") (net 5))
 (segment (start 139.358 49.149) (end 139.358 51.982) (width 0.25) (layer "F.Cu") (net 5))
 (segment (start 132.207 62.2046) (end 132.207 60.032) (width 0.25) (layer "F.Cu") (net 5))
 (segment (start 135.513676 53.6825) (end 134.7085 53.6825) (width 0.25) (layer "F.Cu") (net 5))
 (segment (start 132.3848 62.3824) (end 133.6606 62.3824) (width 0.25) (layer "F.Cu") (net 5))
 (segment (start 134.581 53.555) (end 134.581 53.467) (width 0.25) (layer "F.Cu") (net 5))
 (segment (start 137.0076 66.3956) (end 137.7052 65.698) (width 0.25) (layer "F.Cu") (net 5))
 (via (at 170.8404 52.5272) (size 0.6) (drill 0.3) (layers "F.Cu" "B.Cu") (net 5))
 (via (at 169.1132 50.6984) (size 0.6) (drill 0.3) (layers "F.Cu" "B.Cu") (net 5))
 (via (at 138.176 48.006) (size 0.6) (drill 0.3) (layers "F.Cu" "B.Cu") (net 5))
 (via (at 167.132 54.4068) (size 0.6) (drill 0.3) (layers "F.Cu" "B.Cu") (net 5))
 (via (at 169.1132 54.4068) (size 0.6) (drill 0.3) (layers "F.Cu" "B.Cu") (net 5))
 (via (at 132.2832 62.2808) (size 0.6) (drill 0.3) (layers "F.Cu" "B.Cu") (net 5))
 (via (at 137.0076 66.3956) (size 0.6) (drill 0.3) (layers "F.Cu" "B.Cu") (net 5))
 (via (at 170.8912 54.4068) (size 0.6) (drill 0.3) (layers "F.Cu" "B.Cu") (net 5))
 (via (at 135.513676 53.6825) (size 0.6) (drill 0.3) (layers "F.Cu" "B.Cu") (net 5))
 (via (at 169.1132 52.4764) (size 0.6) (drill 0.3) (layers "F.Cu" "B.Cu") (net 5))
 (via (at 170.8912 50.6984) (size 0.6) (drill 0.3) (layers "F.Cu" "B.Cu") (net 5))
 (via (at 143.5608 66.294) (size 0.6) (drill 0.3) (layers "F.Cu" "B.Cu") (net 5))
 (via (at 167.132 50.6984) (size 0.6) (drill 0.3) (layers "F.Cu" "B.Cu") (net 5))
 (via (at 167.132 52.5272) (size 0.6) (drill 0.3) (layers "F.Cu" "B.Cu") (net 5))
 (segment (start 135.080086 52.705) (end 131.095 52.705) (width 0.25) (layer "F.Cu") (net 9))
 (segment (start 139.971 53.108) (end 135.483086 53.108) (width 0.25) (layer "F.Cu") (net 9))
 (segment (start 141.046 49.2) (end 141.097 49.149) (width 0.25) (layer "F.Cu") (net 9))
 (segment (start 135.483086 53.108) (end 135.080086 52.705) (width 0.25) (layer "F.Cu") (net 9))
 (segment (start 131.095 52.705) (end 129.8 54) (width 0.25) (layer "F.Cu") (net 9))
 (segment (start 141.046 52.033) (end 139.971 53.108) (width 0.25) (layer "F.Cu") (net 9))
 (segment (start 141.046 52.033) (end 141.046 49.2) (width 0.25) (layer "F.Cu") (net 9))
 (segment (start 137.795 51.435) (end 137.922 51.562) (width 0.25) (layer "F.Cu") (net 14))
 (segment (start 134.581 51.435) (end 137.795 51.435) (width 0.25) (layer "F.Cu") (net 14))
 (segment (start 134.454 51.308) (end 134.581 51.435) (width 0.25) (layer "F.Cu") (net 14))
 (segment (start 137.922 51.562) (end 137.922 52.07) (width 0.25) (layer "F.Cu") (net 14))
 (segment (start 137.846 49.581) (end 137.414 49.149) (width 0.25) (layer "F.Cu") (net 14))
 (segment (start 137.846 52.033) (end 137.846 49.581) (width 0.25) (layer "F.Cu") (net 14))
 (segment (start 141.8472 67.31) (end 140.6652 67.31) (width 0.25) (layer "F.Cu") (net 15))
 (segment (start 132.754 54.864) (end 132.754 53.379) (width 0.25) (layer "F.Cu") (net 16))
 (segment (start 132.754 51.308) (end 129.708 51.308) (width 0.25) (layer "F.Cu") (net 10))
 (segment (start 136.9822 68.199) (end 133.999 68.199) (width 0.25) (layer "F.Cu") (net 7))
 (segment (start 137.7188 67.398) (end 139.1412 67.398) (width 0.25) (layer "F.Cu") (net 7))
 (segment (start 137.7188 67.398) (end 137.7188 67.4624) (width 0.25) (layer "F.Cu") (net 7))
 (segment (start 137.7188 67.4624) (end 136.9822 68.199) (width 0.25) (layer "F.Cu") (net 7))
 (segment (start 130.1 64.3) (end 130 64.3) (width 0.25) (layer "F.Cu") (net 7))
 (segment (start 133.999 68.199) (end 130.1 64.3) (width 0.25) (layer "F.Cu") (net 7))
 (segment (start 135.358 57.38) (end 135.358 56.491) (width 1) (layer "F.Cu") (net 1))
 (segment (start 134.402 56.17) (end 135.037 56.17) (width 1) (layer "F.Cu") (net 1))
 (segment (start 137.0035 60.112) (end 137.0035 60.9895) (width 1) (layer "F.Cu") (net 1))
 (segment (start 134.4122 54.767) (end 134.4168 54.767) (width 1) (layer "F.Cu") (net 1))
 (segment (start 135.037 56.17) (end 135.358 56.491) (width 1) (layer "F.Cu") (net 1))
 (segment (start 134.402 54.7772) (end 134.4122 54.767) (width 1) (layer "F.Cu") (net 1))
 (segment (start 137.0035 59.0255) (end 135.358 57.38) (width 1) (layer "F.Cu") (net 1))
 (segment (start 134.402 56.17) (end 130.03 56.17) (width 1) (layer "F.Cu") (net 1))
 (segment (start 137.0035 60.112) (end 137.0035 59.0255) (width 1) (layer "F.Cu") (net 1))
 (segment (start 134.402 56.17) (end 134.402 54.7772) (width 1) (layer "F.Cu") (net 1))
 (segment (start 130.03 56.17) (end 129.9 56.3) (width 1) (layer "F.Cu") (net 1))
 (segment (start 135.57 62.373) (end 135.57 60.513) (width 0.25) (layer "F.Cu") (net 4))
 (segment (start 134.913 67.398) (end 134.874 67.437) (width 0.25) (layer "F.Cu") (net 6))
 (segment (start 134.112 64.9732) (end 134.5692 64.516) (width 0.25) (layer "F.Cu") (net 6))
 (segment (start 136.271 67.398) (end 134.913 67.398) (width 0.25) (layer "F.Cu") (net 6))
 (segment (start 134.874 67.398) (end 134.708 67.398) (width 0.25) (layer "F.Cu") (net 6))
 (segment (start 134.112 66.802) (end 134.112 64.9732) (width 0.25) (layer "F.Cu") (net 6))
 (segment (start 134.708 67.398) (end 134.112 66.802) (width 0.25) (layer "F.Cu") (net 6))
 (segment (start 135.001 65.659) (end 136.906 63.754) (width 0.25) (layer "F.Cu") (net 2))
 (segment (start 134.874 65.659) (end 135.001 65.659) (width 0.25) (layer "F.Cu") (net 2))
 (segment (start 136.906 63.754) (end 136.906 62.103) (width 0.25) (layer "F.Cu") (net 2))
 (segment (start 138.4385 61.087) (end 138.4385 56.9045) (width 1) (layer "F.Cu") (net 3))
 (segment (start 138.4385 57.1585) (end 138.176 56.896) (width 0.5) (layer "F.Cu") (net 3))
 (segment (start 139.684 64.135) (end 139.684 61.611) (width 0.25) (layer "F.Cu") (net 3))
 (segment (start 138.4385 56.9045) (end 138.303 56.769) (width 1) (layer "F.Cu") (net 3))
 (segment (start 130.568 58.332) (end 129.9 59) (width 0.25) (layer "F.Cu") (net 8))
 (segment (start 132.207 57.785) (end 132.572 57.42) (width 0.25) (layer "F.Cu") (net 8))
 (segment (start 132.572 57.42) (end 133.858 57.42) (width 0.25) (layer "F.Cu") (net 8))
 (segment (start 132.207 58.332) (end 132.207 57.785) (width 0.25) (layer "F.Cu") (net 8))
 (segment (start 132.207 58.332) (end 130.568 58.332) (width 0.25) (layer "F.Cu") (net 8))
 (segment (start 133.858 59.42) (end 133.858 60.706) (width 0.25) (layer "F.Cu") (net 12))
 (segment (start 133.858 60.706) (end 133.731 60.833) (width 0.25) (layer "F.Cu") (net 12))
 (segment (start 136.398 65.659) (end 137.668 64.389) (width 0.25) (layer "F.Cu") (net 13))
 (segment (start 141.0716 62.992) (end 141.0716 56.9468) (width 1) (layer "F.Cu") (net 11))
 (segment (start 141.1876 63.108) (end 141.0716 62.992) (width 1) (layer "F.Cu") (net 11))
 (segment (start 139.7136 65.698) (end 139.7 65.6844) (width 1) (layer "F.Cu") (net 11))
 (segment (start 141.0716 65.19) (end 141.0716 62.992) (width 1) (layer "F.Cu") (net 11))
 (segment (start 147.392 63.108) (end 168.9752 63.108) (width 1) (layer "F.Cu") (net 11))
 (segment (start 147.373 63.108) (end 141.1876 63.108) (width 1) (layer "F.Cu") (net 11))
 (segment (start 140.5636 65.698) (end 139.7136 65.698) (width 1) (layer "F.Cu") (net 11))
 (segment (start 140.5636 65.698) (end 141.0716 65.19) (width 1) (layer "F.Cu") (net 11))
 (via (at 169.2148 60.7568) (size 0.6) (drill 0.3) (layers "F.Cu" "B.Cu") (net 11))
 (via (at 167.2336 64.4652) (size 0.6) (drill 0.3) (layers "F.Cu" "B.Cu") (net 11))
 (via (at 170.9928 60.7568) (size 0.6) (drill 0.3) (layers "F.Cu" "B.Cu") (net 11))
 (via (at 167.2336 60.7568) (size 0.6) (drill 0.3) (layers "F.Cu" "B.Cu") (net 11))
 (via (at 169.2148 62.5348) (size 0.6) (drill 0.3) (layers "F.Cu" "B.Cu") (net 11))
 (via (at 167.2336 62.5856) (size 0.6) (drill 0.3) (layers "F.Cu" "B.Cu") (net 11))
 (via (at 169.2148 64.4652) (size 0.6) (drill 0.3) (layers "F.Cu" "B.Cu") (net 11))
 (via (at 170.942 62.5856) (size 0.6) (drill 0.3) (layers "F.Cu" "B.Cu") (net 11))
 (via (at 170.9928 64.4652) (size 0.6) (drill 0.3) (layers "F.Cu" "B.Cu") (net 11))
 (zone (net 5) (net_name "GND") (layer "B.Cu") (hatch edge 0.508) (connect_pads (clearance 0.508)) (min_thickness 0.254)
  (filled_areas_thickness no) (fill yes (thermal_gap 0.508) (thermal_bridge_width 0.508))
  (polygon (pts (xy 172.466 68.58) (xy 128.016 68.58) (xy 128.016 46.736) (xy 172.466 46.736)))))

